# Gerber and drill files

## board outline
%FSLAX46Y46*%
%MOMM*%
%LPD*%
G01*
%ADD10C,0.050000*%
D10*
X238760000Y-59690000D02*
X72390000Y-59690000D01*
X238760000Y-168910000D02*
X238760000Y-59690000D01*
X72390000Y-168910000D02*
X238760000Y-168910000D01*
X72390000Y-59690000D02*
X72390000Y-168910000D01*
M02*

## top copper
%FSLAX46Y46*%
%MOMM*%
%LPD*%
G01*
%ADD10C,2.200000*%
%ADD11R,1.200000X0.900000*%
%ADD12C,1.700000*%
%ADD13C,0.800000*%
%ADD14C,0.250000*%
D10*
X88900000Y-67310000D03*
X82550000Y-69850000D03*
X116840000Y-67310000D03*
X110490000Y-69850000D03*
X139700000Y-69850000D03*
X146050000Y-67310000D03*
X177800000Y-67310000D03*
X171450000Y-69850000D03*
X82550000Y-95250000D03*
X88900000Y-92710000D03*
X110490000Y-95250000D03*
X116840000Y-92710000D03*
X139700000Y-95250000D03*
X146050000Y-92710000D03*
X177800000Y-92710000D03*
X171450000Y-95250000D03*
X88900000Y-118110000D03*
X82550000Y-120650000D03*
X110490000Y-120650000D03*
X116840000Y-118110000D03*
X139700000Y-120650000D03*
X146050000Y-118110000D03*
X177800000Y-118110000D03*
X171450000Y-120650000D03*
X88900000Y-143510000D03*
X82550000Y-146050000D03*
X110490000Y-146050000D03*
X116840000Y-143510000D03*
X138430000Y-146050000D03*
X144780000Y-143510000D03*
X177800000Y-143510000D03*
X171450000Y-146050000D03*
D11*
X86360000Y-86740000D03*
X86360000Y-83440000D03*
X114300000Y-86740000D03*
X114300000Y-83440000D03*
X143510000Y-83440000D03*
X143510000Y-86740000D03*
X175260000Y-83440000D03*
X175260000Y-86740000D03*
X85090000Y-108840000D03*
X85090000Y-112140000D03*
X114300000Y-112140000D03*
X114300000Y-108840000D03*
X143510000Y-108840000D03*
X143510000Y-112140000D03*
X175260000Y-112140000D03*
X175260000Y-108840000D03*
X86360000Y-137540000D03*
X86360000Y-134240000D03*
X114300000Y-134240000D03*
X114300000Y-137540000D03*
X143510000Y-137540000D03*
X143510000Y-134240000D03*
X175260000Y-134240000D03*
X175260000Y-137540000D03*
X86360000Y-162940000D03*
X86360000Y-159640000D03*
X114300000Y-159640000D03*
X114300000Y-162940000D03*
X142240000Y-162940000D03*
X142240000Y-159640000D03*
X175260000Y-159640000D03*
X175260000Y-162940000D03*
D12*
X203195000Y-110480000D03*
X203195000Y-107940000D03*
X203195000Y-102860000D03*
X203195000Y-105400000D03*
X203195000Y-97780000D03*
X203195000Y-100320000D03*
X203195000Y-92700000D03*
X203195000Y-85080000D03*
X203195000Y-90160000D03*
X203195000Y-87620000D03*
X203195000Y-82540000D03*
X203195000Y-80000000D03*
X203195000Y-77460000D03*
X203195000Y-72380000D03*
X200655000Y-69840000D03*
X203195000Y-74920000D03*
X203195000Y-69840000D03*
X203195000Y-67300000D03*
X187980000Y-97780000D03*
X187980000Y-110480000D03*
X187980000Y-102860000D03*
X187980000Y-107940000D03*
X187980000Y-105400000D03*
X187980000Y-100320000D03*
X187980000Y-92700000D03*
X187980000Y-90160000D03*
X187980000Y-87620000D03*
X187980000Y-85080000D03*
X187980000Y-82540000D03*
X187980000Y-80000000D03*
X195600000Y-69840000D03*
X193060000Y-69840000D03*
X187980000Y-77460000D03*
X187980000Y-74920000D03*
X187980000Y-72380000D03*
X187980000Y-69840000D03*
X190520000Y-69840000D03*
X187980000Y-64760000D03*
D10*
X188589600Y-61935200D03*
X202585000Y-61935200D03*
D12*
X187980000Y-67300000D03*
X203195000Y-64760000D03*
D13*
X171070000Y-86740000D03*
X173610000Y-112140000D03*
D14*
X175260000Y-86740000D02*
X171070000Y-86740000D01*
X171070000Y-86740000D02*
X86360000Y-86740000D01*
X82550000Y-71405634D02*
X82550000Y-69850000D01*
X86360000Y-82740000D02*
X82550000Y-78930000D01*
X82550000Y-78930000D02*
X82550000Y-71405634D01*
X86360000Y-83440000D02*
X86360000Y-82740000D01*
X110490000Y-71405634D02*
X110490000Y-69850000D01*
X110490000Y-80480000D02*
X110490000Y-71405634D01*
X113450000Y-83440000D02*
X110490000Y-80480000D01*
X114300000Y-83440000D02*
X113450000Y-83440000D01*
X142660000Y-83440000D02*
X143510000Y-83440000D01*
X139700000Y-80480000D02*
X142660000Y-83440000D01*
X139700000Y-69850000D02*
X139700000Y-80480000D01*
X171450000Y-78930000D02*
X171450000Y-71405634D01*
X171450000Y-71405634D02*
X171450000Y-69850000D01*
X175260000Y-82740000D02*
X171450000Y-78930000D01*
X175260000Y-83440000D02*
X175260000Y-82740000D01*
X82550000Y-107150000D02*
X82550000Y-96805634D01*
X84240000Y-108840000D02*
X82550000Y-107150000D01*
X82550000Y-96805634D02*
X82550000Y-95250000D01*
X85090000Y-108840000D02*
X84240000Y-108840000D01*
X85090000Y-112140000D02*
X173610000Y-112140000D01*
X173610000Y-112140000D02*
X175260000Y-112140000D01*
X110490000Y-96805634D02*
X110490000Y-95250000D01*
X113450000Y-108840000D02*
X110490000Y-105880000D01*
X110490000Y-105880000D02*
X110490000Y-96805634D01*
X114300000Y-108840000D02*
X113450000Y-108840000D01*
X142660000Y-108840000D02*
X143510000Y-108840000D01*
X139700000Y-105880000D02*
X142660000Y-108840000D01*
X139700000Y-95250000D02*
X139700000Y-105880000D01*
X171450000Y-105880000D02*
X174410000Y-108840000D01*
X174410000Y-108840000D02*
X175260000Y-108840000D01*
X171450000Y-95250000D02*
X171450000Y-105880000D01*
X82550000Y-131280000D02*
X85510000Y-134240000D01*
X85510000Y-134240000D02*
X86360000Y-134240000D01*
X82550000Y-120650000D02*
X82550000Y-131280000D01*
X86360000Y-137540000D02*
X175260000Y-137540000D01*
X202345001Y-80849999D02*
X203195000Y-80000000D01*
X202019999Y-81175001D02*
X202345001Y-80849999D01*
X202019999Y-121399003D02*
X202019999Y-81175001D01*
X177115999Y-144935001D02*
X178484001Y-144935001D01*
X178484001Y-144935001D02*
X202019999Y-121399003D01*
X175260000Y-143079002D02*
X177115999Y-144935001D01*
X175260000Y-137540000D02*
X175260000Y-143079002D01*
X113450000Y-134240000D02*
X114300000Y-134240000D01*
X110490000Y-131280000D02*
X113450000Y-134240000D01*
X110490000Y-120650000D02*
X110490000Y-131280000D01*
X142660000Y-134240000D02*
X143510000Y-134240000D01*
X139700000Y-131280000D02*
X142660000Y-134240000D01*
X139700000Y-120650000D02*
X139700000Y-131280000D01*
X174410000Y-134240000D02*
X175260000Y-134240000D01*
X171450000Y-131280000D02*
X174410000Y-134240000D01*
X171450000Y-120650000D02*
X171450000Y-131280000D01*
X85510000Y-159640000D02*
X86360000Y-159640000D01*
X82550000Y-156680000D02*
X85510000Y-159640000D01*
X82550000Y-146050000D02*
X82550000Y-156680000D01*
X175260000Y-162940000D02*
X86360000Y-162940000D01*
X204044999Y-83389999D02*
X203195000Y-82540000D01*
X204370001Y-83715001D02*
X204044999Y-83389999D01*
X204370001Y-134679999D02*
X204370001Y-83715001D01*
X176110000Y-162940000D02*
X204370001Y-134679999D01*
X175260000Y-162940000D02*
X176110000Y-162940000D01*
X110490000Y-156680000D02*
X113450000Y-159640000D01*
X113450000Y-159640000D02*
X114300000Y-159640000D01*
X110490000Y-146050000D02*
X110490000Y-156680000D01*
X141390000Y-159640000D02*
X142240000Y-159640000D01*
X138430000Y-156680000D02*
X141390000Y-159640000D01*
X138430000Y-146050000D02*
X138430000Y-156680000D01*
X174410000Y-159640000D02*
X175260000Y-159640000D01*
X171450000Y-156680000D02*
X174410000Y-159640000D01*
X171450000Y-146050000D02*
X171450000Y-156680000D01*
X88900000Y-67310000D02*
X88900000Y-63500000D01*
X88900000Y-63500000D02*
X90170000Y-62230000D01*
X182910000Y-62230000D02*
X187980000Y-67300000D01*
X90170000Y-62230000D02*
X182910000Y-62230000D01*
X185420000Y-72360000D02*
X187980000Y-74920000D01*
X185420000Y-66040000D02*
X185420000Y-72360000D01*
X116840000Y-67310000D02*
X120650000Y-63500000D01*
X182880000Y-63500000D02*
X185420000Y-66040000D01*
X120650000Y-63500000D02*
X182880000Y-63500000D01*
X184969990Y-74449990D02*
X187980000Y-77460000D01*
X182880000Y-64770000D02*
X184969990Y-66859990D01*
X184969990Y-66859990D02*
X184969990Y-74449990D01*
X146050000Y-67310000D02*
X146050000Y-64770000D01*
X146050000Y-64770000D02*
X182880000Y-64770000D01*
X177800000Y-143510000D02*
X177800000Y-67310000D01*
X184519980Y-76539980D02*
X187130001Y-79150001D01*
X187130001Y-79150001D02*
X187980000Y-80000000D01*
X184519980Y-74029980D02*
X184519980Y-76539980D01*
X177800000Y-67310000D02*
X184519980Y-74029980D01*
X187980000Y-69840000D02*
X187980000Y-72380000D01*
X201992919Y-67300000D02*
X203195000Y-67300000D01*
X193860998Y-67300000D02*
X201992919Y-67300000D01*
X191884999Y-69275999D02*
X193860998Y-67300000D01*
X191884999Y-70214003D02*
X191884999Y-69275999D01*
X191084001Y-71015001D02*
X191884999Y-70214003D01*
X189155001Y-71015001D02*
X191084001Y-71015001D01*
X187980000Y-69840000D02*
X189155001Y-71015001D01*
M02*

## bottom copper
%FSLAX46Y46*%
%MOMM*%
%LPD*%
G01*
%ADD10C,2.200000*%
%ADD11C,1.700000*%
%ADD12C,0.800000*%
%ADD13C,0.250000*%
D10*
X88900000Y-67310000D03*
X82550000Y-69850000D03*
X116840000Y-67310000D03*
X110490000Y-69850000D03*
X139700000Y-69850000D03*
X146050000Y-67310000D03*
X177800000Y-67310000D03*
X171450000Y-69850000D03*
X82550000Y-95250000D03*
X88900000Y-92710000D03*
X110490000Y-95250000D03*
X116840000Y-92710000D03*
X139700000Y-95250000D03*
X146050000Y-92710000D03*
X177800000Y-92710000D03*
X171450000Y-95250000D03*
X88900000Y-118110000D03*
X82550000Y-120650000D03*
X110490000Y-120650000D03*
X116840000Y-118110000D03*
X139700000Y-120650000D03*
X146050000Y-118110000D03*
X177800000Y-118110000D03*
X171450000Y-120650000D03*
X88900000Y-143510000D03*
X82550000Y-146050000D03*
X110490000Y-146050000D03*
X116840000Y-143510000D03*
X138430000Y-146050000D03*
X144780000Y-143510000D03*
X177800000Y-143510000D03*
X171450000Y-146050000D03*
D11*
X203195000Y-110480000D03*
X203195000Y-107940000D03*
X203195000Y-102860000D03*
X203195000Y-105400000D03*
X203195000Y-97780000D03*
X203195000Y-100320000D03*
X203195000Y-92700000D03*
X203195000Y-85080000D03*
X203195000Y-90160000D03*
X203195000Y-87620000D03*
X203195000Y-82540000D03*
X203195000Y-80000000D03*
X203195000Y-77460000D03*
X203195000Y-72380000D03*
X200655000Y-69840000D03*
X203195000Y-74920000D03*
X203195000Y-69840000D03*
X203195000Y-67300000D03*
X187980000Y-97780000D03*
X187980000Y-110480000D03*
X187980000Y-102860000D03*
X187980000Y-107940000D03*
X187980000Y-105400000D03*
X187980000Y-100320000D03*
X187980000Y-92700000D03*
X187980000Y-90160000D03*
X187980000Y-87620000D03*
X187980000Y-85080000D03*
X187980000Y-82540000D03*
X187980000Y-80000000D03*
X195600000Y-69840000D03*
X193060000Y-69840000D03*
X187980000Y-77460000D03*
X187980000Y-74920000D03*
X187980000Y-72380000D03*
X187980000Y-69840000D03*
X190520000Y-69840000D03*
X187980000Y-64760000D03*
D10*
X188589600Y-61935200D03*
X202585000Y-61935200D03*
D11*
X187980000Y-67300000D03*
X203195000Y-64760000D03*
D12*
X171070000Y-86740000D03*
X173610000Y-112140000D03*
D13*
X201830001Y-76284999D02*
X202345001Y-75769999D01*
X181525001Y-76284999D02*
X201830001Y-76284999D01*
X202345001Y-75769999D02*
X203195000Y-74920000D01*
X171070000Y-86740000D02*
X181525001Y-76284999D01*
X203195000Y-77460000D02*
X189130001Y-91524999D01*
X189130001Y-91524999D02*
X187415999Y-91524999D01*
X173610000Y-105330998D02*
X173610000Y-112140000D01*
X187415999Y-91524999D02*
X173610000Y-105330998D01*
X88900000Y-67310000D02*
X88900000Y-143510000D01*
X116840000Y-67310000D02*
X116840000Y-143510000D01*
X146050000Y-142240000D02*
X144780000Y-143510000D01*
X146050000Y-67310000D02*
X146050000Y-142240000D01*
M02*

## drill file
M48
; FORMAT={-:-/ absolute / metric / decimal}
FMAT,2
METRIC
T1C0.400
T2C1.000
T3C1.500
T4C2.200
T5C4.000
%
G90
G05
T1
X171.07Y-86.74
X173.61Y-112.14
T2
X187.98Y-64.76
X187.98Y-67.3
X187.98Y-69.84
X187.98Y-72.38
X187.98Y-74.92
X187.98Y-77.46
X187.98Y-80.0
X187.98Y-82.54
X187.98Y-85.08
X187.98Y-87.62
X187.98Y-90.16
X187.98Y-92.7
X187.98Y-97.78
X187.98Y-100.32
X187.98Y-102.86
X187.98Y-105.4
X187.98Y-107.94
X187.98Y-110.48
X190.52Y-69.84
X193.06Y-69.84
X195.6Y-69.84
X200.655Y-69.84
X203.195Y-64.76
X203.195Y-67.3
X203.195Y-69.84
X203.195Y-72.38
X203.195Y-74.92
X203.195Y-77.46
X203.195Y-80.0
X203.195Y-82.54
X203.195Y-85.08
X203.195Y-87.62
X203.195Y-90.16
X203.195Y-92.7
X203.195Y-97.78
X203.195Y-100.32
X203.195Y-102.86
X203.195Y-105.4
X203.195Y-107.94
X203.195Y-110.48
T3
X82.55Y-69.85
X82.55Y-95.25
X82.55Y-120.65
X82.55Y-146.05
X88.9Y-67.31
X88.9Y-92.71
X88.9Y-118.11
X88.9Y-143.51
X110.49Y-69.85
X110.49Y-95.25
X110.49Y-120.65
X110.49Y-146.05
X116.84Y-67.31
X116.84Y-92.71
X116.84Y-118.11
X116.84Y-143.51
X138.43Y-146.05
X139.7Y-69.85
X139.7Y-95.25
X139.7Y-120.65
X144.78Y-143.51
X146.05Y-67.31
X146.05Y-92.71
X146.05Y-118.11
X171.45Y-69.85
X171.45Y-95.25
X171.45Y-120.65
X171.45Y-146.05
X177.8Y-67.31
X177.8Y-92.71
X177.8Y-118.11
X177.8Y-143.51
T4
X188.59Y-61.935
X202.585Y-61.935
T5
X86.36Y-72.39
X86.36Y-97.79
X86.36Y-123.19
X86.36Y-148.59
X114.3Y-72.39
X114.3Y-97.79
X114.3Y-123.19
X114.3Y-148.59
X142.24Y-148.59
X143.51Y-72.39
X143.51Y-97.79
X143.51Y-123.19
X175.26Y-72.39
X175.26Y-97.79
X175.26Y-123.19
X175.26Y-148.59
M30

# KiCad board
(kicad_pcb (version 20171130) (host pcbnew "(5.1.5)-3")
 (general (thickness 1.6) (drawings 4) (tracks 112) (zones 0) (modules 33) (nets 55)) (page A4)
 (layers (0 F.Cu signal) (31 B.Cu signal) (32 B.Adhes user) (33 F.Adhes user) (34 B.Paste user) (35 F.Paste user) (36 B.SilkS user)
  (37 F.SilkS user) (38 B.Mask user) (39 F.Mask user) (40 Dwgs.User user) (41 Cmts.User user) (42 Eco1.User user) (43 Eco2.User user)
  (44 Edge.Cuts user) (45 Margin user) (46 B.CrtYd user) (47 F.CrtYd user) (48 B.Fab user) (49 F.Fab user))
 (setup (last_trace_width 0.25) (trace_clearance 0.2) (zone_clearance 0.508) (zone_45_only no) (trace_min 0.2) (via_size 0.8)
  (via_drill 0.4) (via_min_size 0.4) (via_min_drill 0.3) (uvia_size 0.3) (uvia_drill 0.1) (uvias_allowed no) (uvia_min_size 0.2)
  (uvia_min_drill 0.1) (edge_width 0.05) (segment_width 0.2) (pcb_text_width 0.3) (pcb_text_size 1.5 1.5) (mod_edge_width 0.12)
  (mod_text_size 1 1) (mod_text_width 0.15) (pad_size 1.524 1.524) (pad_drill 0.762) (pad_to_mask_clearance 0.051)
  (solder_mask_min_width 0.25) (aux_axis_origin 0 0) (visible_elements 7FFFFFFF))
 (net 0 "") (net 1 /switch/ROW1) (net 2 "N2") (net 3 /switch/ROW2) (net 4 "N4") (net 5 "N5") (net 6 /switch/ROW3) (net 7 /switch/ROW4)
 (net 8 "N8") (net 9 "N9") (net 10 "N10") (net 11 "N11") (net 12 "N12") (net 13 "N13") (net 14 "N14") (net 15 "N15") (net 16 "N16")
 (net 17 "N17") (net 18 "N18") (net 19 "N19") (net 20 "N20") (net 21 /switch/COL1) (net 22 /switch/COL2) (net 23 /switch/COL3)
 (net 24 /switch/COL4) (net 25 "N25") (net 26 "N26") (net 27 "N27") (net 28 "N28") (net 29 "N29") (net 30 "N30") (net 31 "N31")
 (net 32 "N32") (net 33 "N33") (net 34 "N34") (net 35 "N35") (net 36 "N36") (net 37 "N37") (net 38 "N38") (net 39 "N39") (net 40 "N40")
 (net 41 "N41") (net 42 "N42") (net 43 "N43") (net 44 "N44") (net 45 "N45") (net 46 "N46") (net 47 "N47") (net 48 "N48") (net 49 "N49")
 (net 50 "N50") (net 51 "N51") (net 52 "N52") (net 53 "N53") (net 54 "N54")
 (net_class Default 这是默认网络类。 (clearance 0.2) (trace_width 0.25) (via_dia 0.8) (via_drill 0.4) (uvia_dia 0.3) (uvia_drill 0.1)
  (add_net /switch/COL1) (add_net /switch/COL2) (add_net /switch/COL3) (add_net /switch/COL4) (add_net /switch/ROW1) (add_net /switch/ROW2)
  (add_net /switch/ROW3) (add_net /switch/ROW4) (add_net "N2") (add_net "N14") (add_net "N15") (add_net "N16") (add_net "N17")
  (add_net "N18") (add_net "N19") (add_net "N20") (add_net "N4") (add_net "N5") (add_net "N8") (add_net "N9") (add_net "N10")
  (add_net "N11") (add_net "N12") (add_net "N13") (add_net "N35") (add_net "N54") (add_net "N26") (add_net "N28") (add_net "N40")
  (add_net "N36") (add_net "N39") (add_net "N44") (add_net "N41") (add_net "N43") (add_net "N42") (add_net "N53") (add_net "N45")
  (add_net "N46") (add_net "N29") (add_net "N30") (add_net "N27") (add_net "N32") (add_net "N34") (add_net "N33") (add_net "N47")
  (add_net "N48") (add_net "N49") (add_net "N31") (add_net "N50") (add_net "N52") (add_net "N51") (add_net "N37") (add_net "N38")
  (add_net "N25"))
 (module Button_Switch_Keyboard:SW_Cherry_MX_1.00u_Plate (layer F.Cu) (at 88.9 67.31)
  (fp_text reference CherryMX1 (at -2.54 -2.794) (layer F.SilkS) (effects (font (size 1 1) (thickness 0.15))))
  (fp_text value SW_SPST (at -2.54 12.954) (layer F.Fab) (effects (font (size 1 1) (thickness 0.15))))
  (pad 1 thru_hole circle (at 0 0) (size 2.2 2.2) (drill 1.5) (layers *.Cu *.Mask) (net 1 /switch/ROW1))
  (pad 2 thru_hole circle (at -6.35 2.54) (size 2.2 2.2) (drill 1.5) (layers *.Cu *.Mask) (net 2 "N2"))
  (pad "" np_thru_hole circle (at -2.54 5.08) (size 4 4) (drill 4) (layers *.Cu *.Mask)))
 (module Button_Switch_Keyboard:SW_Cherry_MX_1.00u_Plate (layer F.Cu) (at 116.84 67.31)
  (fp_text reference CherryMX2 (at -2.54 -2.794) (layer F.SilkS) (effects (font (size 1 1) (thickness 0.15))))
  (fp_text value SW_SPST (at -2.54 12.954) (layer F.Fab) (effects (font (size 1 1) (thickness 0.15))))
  (pad 1 thru_hole circle (at 0 0) (size 2.2 2.2) (drill 1.5) (layers *.Cu *.Mask) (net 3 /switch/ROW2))
  (pad 2 thru_hole circle (at -6.35 2.54) (size 2.2 2.2) (drill 1.5) (layers *.Cu *.Mask) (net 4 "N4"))
  (pad "" np_thru_hole circle (at -2.54 5.08) (size 4 4) (drill 4) (layers *.Cu *.Mask)))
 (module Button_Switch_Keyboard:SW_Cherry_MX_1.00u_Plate (layer F.Cu) (at 146.05 67.31)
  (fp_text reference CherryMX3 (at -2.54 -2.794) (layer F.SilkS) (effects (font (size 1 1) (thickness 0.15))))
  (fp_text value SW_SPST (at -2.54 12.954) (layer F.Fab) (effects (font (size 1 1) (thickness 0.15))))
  (pad "" np_thru_hole circle (at -2.54 5.08) (size 4 4) (drill 4) (layers *.Cu *.Mask))
  (pad 2 thru_hole circle (at -6.35 2.54) (size 2.2 2.2) (drill 1.5) (layers *.Cu *.Mask) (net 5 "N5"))
  (pad 1 thru_hole circle (at 0 0) (size 2.2 2.2) (drill 1.5) (layers *.Cu *.Mask) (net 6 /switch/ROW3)))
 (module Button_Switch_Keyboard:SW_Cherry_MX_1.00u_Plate (layer F.Cu) (at 177.8 67.31)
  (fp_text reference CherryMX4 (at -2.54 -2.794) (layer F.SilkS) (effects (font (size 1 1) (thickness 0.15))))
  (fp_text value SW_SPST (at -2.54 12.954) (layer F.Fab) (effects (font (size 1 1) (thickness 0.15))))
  (pad 1 thru_hole circle (at 0 0) (size 2.2 2.2) (drill 1.5) (layers *.Cu *.Mask) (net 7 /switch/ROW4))
  (pad 2 thru_hole circle (at -6.35 2.54) (size 2.2 2.2) (drill 1.5) (layers *.Cu *.Mask) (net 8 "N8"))
  (pad "" np_thru_hole circle (at -2.54 5.08) (size 4 4) (drill 4) (layers *.Cu *.Mask)))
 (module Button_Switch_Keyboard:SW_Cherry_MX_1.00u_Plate (layer F.Cu) (at 88.9 92.71)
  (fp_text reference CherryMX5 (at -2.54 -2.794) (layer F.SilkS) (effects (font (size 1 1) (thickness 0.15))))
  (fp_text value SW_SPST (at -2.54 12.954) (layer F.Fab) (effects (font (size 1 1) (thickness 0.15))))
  (pad "" np_thru_hole circle (at -2.54 5.08) (size 4 4) (drill 4) (layers *.Cu *.Mask))
  (pad 2 thru_hole circle (at -6.35 2.54) (size 2.2 2.2) (drill 1.5) (layers *.Cu *.Mask) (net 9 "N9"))
  (pad 1 thru_hole circle (at 0 0) (size 2.2 2.2) (drill 1.5) (layers *.Cu *.Mask) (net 1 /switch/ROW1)))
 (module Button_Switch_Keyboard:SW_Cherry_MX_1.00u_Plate (layer F.Cu) (at 116.84 92.71)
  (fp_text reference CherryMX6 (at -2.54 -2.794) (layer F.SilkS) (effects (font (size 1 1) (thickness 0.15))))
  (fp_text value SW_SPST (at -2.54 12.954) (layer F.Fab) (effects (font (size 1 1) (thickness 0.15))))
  (pad "" np_thru_hole circle (at -2.54 5.08) (size 4 4) (drill 4) (layers *.Cu *.Mask))
  (pad 2 thru_hole circle (at -6.35 2.54) (size 2.2 2.2) (drill 1.5) (layers *.Cu *.Mask) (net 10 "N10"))
  (pad 1 thru_hole circle (at 0 0) (size 2.2 2.2) (drill 1.5) (layers *.Cu *.Mask) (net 3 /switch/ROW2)))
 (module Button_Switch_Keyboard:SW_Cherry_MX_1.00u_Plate (layer F.Cu) (at 146.05 92.71)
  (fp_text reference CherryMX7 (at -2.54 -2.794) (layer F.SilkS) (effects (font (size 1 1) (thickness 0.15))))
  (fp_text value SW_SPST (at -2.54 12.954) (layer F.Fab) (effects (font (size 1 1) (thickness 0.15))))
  (pad "" np_thru_hole circle (at -2.54 5.08) (size 4 4) (drill 4) (layers *.Cu *.Mask))
  (pad 2 thru_hole circle (at -6.35 2.54) (size 2.2 2.2) (drill 1.5) (layers *.Cu *.Mask) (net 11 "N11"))
  (pad 1 thru_hole circle (at 0 0) (size 2.2 2.2) (drill 1.5) (layers *.Cu *.Mask) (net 6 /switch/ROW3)))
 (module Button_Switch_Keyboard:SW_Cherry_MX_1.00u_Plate (layer F.Cu) (at 177.8 92.71)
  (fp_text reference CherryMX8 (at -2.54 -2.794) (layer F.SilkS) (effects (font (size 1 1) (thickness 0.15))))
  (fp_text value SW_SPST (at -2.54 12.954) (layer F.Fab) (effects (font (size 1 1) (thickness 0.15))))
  (pad 1 thru_hole circle (at 0 0) (size 2.2 2.2) (drill 1.5) (layers *.Cu *.Mask) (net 7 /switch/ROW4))
  (pad 2 thru_hole circle (at -6.35 2.54) (size 2.2 2.2) (drill 1.5) (layers *.Cu *.Mask) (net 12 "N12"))
  (pad "" np_thru_hole circle (at -2.54 5.08) (size 4 4) (drill 4) (layers *.Cu *.Mask)))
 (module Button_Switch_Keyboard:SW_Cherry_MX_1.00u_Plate (layer F.Cu) (at 88.9 118.11)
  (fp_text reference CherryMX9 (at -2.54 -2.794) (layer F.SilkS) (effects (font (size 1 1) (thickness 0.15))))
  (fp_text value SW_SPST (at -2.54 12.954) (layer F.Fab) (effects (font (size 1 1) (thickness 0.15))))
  (pad 1 thru_hole circle (at 0 0) (size 2.2 2.2) (drill 1.5) (layers *.Cu *.Mask) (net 1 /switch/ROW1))
  (pad 2 thru_hole circle (at -6.35 2.54) (size 2.2 2.2) (drill 1.5) (layers *.Cu *.Mask) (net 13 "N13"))
  (pad "" np_thru_hole circle (at -2.54 5.08) (size 4 4) (drill 4) (layers *.Cu *.Mask)))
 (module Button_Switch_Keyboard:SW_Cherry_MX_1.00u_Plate (layer F.Cu) (at 116.84 118.11)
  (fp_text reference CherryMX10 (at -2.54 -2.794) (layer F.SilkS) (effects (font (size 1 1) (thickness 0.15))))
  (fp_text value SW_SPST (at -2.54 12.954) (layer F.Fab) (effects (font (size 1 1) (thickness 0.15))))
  (pad "" np_thru_hole circle (at -2.54 5.08) (size 4 4) (drill 4) (layers *.Cu *.Mask))
  (pad 2 thru_hole circle (at -6.35 2.54) (size 2.2 2.2) (drill 1.5) (layers *.Cu *.Mask) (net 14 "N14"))
  (pad 1 thru_hole circle (at 0 0) (size 2.2 2.2) (drill 1.5) (layers *.Cu *.Mask) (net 3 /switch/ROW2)))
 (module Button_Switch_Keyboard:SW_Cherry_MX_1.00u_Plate (layer F.Cu) (at 146.05 118.11)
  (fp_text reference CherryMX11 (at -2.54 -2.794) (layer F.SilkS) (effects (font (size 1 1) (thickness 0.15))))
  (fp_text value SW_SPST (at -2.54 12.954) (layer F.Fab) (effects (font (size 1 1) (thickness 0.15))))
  (pad "" np_thru_hole circle (at -2.54 5.08) (size 4 4) (drill 4) (layers *.Cu *.Mask))
  (pad 2 thru_hole circle (at -6.35 2.54) (size 2.2 2.2) (drill 1.5) (layers *.Cu *.Mask) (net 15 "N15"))
  (pad 1 thru_hole circle (at 0 0) (size 2.2 2.2) (drill 1.5) (layers *.Cu *.Mask) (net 6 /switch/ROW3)))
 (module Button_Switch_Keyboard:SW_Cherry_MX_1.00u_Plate (layer F.Cu) (at 177.8 118.11)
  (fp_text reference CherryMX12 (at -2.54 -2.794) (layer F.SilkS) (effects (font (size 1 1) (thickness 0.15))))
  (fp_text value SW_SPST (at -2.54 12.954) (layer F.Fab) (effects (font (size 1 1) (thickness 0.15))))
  (pad 1 thru_hole circle (at 0 0) (size 2.2 2.2) (drill 1.5) (layers *.Cu *.Mask) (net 7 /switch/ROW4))
  (pad 2 thru_hole circle (at -6.35 2.54) (size 2.2 2.2) (drill 1.5) (layers *.Cu *.Mask) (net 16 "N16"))
  (pad "" np_thru_hole circle (at -2.54 5.08) (size 4 4) (drill 4) (layers *.Cu *.Mask)))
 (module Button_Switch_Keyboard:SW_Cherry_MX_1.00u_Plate (layer F.Cu) (at 88.9 143.51)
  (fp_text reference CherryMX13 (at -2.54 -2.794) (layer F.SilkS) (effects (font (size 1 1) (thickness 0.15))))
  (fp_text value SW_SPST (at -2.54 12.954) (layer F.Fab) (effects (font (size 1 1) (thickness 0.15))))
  (pad 1 thru_hole circle (at 0 0) (size 2.2 2.2) (drill 1.5) (layers *.Cu *.Mask) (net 1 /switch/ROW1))
  (pad 2 thru_hole circle (at -6.35 2.54) (size 2.2 2.2) (drill 1.5) (layers *.Cu *.Mask) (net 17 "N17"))
  (pad "" np_thru_hole circle (at -2.54 5.08) (size 4 4) (drill 4) (layers *.Cu *.Mask)))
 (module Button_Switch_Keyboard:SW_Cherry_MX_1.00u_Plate (layer F.Cu) (at 116.84 143.51)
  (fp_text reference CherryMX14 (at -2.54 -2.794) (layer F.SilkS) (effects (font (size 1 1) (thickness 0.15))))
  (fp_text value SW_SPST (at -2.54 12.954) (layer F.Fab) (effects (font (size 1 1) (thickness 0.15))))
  (pad "" np_thru_hole circle (at -2.54 5.08) (size 4 4) (drill 4) (layers *.Cu *.Mask))
  (pad 2 thru_hole circle (at -6.35 2.54) (size 2.2 2.2) (drill 1.5) (layers *.Cu *.Mask) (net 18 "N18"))
  (pad 1 thru_hole circle (at 0 0) (size 2.2 2.2) (drill 1.5) (layers *.Cu *.Mask) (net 3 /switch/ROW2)))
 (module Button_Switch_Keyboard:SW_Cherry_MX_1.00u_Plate (layer F.Cu) (at 144.78 143.51)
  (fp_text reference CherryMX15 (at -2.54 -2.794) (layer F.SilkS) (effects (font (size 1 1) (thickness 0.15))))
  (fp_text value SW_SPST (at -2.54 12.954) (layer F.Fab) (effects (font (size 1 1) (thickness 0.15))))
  (pad "" np_thru_hole circle (at -2.54 5.08) (size 4 4) (drill 4) (layers *.Cu *.Mask))
  (pad 2 thru_hole circle (at -6.35 2.54) (size 2.2 2.2) (drill 1.5) (layers *.Cu *.Mask) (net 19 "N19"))
  (pad 1 thru_hole circle (at 0 0) (size 2.2 2.2) (drill 1.5) (layers *.Cu *.Mask) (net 6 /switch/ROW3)))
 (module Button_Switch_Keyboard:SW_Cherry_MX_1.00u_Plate (layer F.Cu) (at 177.8 143.51)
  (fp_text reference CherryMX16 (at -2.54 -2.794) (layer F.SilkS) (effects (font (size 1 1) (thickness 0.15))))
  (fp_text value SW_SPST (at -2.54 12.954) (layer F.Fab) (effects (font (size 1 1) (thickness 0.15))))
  (pad 1 thru_hole circle (at 0 0) (size 2.2 2.2) (drill 1.5) (layers *.Cu *.Mask) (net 7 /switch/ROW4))
  (pad 2 thru_hole circle (at -6.35 2.54) (size 2.2 2.2) (drill 1.5) (layers *.Cu *.Mask) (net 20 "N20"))
  (pad "" np_thru_hole circle (at -2.54 5.08) (size 4 4) (drill 4) (layers *.Cu *.Mask)))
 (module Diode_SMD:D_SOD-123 (layer F.Cu) (at 86.36 85.09 90)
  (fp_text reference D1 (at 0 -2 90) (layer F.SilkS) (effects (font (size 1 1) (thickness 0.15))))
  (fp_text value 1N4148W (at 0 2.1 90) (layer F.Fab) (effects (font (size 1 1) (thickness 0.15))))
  (pad 1 smd rect (at -1.65 0 90) (size 0.9 1.2) (layers F.Cu F.Paste F.Mask) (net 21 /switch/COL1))
  (pad 2 smd rect (at 1.65 0 90) (size 0.9 1.2) (layers F.Cu F.Paste F.Mask) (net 2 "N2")))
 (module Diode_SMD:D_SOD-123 (layer F.Cu) (at 114.3 85.09 90)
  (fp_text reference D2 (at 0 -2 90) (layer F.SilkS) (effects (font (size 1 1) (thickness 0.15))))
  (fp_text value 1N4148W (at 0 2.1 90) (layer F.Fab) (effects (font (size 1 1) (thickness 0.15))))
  (pad 1 smd rect (at -1.65 0 90) (size 0.9 1.2) (layers F.Cu F.Paste F.Mask) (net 21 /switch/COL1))
  (pad 2 smd rect (at 1.65 0 90) (size 0.9 1.2) (layers F.Cu F.Paste F.Mask) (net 4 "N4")))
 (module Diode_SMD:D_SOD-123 (layer F.Cu) (at 143.51 85.09 90)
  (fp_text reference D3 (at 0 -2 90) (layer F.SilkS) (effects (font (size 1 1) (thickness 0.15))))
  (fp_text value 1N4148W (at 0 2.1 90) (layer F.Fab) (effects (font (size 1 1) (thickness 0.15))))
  (pad 2 smd rect (at 1.65 0 90) (size 0.9 1.2) (layers F.Cu F.Paste F.Mask) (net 5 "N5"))
  (pad 1 smd rect (at -1.65 0 90) (size 0.9 1.2) (layers F.Cu F.Paste F.Mask) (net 21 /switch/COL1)))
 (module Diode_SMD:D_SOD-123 (layer F.Cu) (at 175.26 85.09 90)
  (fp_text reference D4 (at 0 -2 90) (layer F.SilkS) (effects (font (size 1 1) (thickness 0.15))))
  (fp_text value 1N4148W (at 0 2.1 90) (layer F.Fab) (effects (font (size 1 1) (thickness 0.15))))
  (pad 2 smd rect (at 1.65 0 90) (size 0.9 1.2) (layers F.Cu F.Paste F.Mask) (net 8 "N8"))
  (pad 1 smd rect (at -1.65 0 90) (size 0.9 1.2) (layers F.Cu F.Paste F.Mask) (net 21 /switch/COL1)))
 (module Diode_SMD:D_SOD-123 (layer F.Cu) (at 85.09 110.49 90)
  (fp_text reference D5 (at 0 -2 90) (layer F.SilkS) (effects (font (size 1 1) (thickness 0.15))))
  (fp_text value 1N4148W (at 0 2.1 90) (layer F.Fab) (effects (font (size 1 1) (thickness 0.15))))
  (pad 2 smd rect (at 1.65 0 90) (size 0.9 1.2) (layers F.Cu F.Paste F.Mask) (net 9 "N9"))
  (pad 1 smd rect (at -1.65 0 90) (size 0.9 1.2) (layers F.Cu F.Paste F.Mask) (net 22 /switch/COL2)))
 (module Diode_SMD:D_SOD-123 (layer F.Cu) (at 114.3 110.49 90)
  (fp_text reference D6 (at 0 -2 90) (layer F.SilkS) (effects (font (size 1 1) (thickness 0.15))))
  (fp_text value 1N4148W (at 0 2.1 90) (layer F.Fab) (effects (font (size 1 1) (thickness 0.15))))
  (pad 1 smd rect (at -1.65 0 90) (size 0.9 1.2) (layers F.Cu F.Paste F.Mask) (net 22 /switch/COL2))
  (pad 2 smd rect (at 1.65 0 90) (size 0.9 1.2) (layers F.Cu F.Paste F.Mask) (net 10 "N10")))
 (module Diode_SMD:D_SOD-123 (layer F.Cu) (at 143.51 110.49 90)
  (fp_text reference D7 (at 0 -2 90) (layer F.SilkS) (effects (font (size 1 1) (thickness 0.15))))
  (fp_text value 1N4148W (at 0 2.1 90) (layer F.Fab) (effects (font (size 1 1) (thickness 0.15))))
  (pad 2 smd rect (at 1.65 0 90) (size 0.9 1.2) (layers F.Cu F.Paste F.Mask) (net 11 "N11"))
  (pad 1 smd rect (at -1.65 0 90) (size 0.9 1.2) (layers F.Cu F.Paste F.Mask) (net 22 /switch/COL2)))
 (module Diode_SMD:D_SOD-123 (layer F.Cu) (at 175.26 110.49 90)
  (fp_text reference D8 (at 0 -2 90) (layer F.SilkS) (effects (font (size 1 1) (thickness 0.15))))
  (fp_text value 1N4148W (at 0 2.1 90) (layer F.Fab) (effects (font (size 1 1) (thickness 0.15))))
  (pad 1 smd rect (at -1.65 0 90) (size 0.9 1.2) (layers F.Cu F.Paste F.Mask) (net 22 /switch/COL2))
  (pad 2 smd rect (at 1.65 0 90) (size 0.9 1.2) (layers F.Cu F.Paste F.Mask) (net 12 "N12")))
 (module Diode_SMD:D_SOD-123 (layer F.Cu) (at 86.36 135.89 90)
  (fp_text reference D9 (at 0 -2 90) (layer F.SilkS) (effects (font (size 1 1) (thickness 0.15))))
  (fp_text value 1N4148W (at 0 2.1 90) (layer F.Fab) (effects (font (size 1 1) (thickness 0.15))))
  (pad 1 smd rect (at -1.65 0 90) (size 0.9 1.2) (layers F.Cu F.Paste F.Mask) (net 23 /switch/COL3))
  (pad 2 smd rect (at 1.65 0 90) (size 0.9 1.2) (layers F.Cu F.Paste F.Mask) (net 13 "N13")))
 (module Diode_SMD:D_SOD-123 (layer F.Cu) (at 114.3 135.89 90)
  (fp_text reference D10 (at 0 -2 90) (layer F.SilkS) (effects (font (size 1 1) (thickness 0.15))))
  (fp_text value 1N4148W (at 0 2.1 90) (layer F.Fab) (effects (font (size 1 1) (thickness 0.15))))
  (pad 2 smd rect (at 1.65 0 90) (size 0.9 1.2) (layers F.Cu F.Paste F.Mask) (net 14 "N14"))
  (pad 1 smd rect (at -1.65 0 90) (size 0.9 1.2) (layers F.Cu F.Paste F.Mask) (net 23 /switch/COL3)))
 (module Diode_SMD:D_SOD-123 (layer F.Cu) (at 143.51 135.89 90)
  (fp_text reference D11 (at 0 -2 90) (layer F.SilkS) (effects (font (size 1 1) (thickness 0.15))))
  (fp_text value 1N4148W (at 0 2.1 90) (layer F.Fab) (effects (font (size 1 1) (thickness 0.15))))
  (pad 1 smd rect (at -1.65 0 90) (size 0.9 1.2) (layers F.Cu F.Paste F.Mask) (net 23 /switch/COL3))
  (pad 2 smd rect (at 1.65 0 90) (size 0.9 1.2) (layers F.Cu F.Paste F.Mask) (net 15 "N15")))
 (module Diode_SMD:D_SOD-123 (layer F.Cu) (at 175.26 135.89 90)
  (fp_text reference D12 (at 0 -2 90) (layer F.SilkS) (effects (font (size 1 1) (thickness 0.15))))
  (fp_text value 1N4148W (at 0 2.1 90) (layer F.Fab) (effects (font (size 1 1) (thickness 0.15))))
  (pad 2 smd rect (at 1.65 0 90) (size 0.9 1.2) (layers F.Cu F.Paste F.Mask) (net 16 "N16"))
  (pad 1 smd rect (at -1.65 0 90) (size 0.9 1.2) (layers F.Cu F.Paste F.Mask) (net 23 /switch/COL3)))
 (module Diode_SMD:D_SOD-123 (layer F.Cu) (at 86.36 161.29 90)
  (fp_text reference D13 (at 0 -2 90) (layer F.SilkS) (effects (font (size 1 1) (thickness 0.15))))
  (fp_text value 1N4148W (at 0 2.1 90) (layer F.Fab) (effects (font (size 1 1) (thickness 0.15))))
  (pad 1 smd rect (at -1.65 0 90) (size 0.9 1.2) (layers F.Cu F.Paste F.Mask) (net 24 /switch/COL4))
  (pad 2 smd rect (at 1.65 0 90) (size 0.9 1.2) (layers F.Cu F.Paste F.Mask) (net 17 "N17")))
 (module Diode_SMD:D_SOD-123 (layer F.Cu) (at 114.3 161.29 90)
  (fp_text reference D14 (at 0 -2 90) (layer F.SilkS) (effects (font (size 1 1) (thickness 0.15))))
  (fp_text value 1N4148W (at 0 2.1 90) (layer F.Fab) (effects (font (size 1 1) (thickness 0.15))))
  (pad 2 smd rect (at 1.65 0 90) (size 0.9 1.2) (layers F.Cu F.Paste F.Mask) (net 18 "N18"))
  (pad 1 smd rect (at -1.65 0 90) (size 0.9 1.2) (layers F.Cu F.Paste F.Mask) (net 24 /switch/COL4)))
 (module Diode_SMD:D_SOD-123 (layer F.Cu) (at 142.24 161.29 90)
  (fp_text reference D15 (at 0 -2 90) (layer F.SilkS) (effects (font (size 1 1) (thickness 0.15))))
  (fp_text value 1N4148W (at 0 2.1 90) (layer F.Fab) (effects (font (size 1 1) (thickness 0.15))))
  (pad 1 smd rect (at -1.65 0 90) (size 0.9 1.2) (layers F.Cu F.Paste F.Mask) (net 24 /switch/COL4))
  (pad 2 smd rect (at 1.65 0 90) (size 0.9 1.2) (layers F.Cu F.Paste F.Mask) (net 19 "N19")))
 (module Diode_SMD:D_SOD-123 (layer F.Cu) (at 175.26 161.29 90)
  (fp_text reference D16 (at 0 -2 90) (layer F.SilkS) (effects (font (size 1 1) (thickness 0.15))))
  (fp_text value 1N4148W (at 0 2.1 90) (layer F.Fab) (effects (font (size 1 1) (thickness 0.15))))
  (pad 2 smd rect (at 1.65 0 90) (size 0.9 1.2) (layers F.Cu F.Paste F.Mask) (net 20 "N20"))
  (pad 1 smd rect (at -1.65 0 90) (size 0.9 1.2) (layers F.Cu F.Paste F.Mask) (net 24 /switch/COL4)))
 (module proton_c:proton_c (layer F.Cu) (at 195.58 80.01)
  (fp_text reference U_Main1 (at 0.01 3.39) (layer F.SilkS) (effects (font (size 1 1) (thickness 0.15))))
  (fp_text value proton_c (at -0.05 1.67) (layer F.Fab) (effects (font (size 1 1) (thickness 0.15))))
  (pad RST thru_hole circle (at 7.615 30.47) (size 1.7 1.7) (drill 1) (layers *.Cu *.Mask) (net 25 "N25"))
  (pad A13 thru_hole circle (at 7.615 27.93) (size 1.7 1.7) (drill 1) (layers *.Cu *.Mask) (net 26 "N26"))
  (pad B12 thru_hole circle (at 7.615 22.85) (size 1.7 1.7) (drill 1) (layers *.Cu *.Mask) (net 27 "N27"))
  (pad A14 thru_hole circle (at 7.615 25.39) (size 1.7 1.7) (drill 1) (layers *.Cu *.Mask) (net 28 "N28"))
  (pad B10 thru_hole circle (at 7.615 17.77) (size 1.7 1.7) (drill 1) (layers *.Cu *.Mask) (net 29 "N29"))
  (pad B11 thru_hole circle (at 7.615 20.31) (size 1.7 1.7) (drill 1) (layers *.Cu *.Mask) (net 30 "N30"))
  (pad B9 thru_hole circle (at 7.615 12.69) (size 1.7 1.7) (drill 1) (layers *.Cu *.Mask) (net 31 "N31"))
  (pad B13 thru_hole circle (at 7.615 5.07) (size 1.7 1.7) (drill 1) (layers *.Cu *.Mask) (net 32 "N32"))
  (pad B15 thru_hole circle (at 7.615 10.15) (size 1.7 1.7) (drill 1) (layers *.Cu *.Mask) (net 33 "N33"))
  (pad B14 thru_hole circle (at 7.615 7.61) (size 1.7 1.7) (drill 1) (layers *.Cu *.Mask) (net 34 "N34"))
  (pad B8 thru_hole circle (at 7.615 2.53) (size 1.7 1.7) (drill 1) (layers *.Cu *.Mask) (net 24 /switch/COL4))
  (pad A0 thru_hole circle (at 7.615 -0.01) (size 1.7 1.7) (drill 1) (layers *.Cu *.Mask) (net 23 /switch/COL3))
  (pad A1 thru_hole circle (at 7.615 -2.55) (size 1.7 1.7) (drill 1) (layers *.Cu *.Mask) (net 22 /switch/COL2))
  (pad 3.3V thru_hole circle (at 7.615 -7.63) (size 1.7 1.7) (drill 1) (layers *.Cu *.Mask) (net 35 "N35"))
  (pad A3|5v thru_hole circle (at 5.075 -10.17) (size 1.7 1.7) (drill 1) (layers *.Cu *.Mask) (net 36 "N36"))
  (pad A2 thru_hole circle (at 7.615 -5.09) (size 1.7 1.7) (drill 1) (layers *.Cu *.Mask) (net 21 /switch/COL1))
  (pad DFU thru_hole circle (at 7.615 -10.17) (size 1.7 1.7) (drill 1) (layers *.Cu *.Mask) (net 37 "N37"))
  (pad GND thru_hole circle (at 7.615 -12.71) (size 1.7 1.7) (drill 1) (layers *.Cu *.Mask) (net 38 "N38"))
  (pad A4 thru_hole circle (at -7.6 17.77) (size 1.7 1.7) (drill 1) (layers *.Cu *.Mask) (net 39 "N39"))
  (pad A15 thru_hole circle (at -7.6 30.47) (size 1.7 1.7) (drill 1) (layers *.Cu *.Mask) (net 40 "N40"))
  (pad A6 thru_hole circle (at -7.6 22.85) (size 1.7 1.7) (drill 1) (layers *.Cu *.Mask) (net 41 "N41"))
  (pad A8 thru_hole circle (at -7.6 27.93) (size 1.7 1.7) (drill 1) (layers *.Cu *.Mask) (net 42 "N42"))
  (pad A7 thru_hole circle (at -7.6 25.39) (size 1.7 1.7) (drill 1) (layers *.Cu *.Mask) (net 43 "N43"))
  (pad A5 thru_hole circle (at -7.6 20.31) (size 1.7 1.7) (drill 1) (layers *.Cu *.Mask) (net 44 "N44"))
  (pad B0 thru_hole circle (at -7.6 12.69) (size 1.7 1.7) (drill 1) (layers *.Cu *.Mask) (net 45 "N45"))
  (pad B1 thru_hole circle (at -7.6 10.15) (size 1.7 1.7) (drill 1) (layers *.Cu *.Mask) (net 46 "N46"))
  (pad B2 thru_hole circle (at -7.6 7.61) (size 1.7 1.7) (drill 1) (layers *.Cu *.Mask) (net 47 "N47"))
  (pad B3 thru_hole circle (at -7.6 5.07) (size 1.7 1.7) (drill 1) (layers *.Cu *.Mask) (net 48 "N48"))
  (pad B4 thru_hole circle (at -7.6 2.53) (size 1.7 1.7) (drill 1) (layers *.Cu *.Mask) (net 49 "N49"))
  (pad B5 thru_hole circle (at -7.6 -0.01) (size 1.7 1.7) (drill 1) (layers *.Cu *.Mask) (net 7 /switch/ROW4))
  (pad CHRG thru_hole circle (at 0.02 -10.17) (size 1.7 1.7) (drill 1) (layers *.Cu *.Mask) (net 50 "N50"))
  (pad D- thru_hole circle (at -2.52 -10.17) (size 1.7 1.7) (drill 1) (layers *.Cu *.Mask) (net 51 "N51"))
  (pad B6 thru_hole circle (at -7.6 -2.55) (size 1.7 1.7) (drill 1) (layers *.Cu *.Mask) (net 6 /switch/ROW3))
  (pad B7 thru_hole circle (at -7.6 -5.09) (size 1.7 1.7) (drill 1) (layers *.Cu *.Mask) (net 3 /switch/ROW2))
  (pad GND thru_hole circle (at -7.6 -7.63) (size 1.7 1.7) (drill 1) (layers *.Cu *.Mask) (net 38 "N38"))
  (pad GND thru_hole circle (at -7.6 -10.17) (size 1.7 1.7) (drill 1) (layers *.Cu *.Mask) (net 38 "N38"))
  (pad D+ thru_hole circle (at -5.06 -10.17) (size 1.7 1.7) (drill 1) (layers *.Cu *.Mask) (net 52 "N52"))
  (pad A9 thru_hole circle (at -7.6 -15.25) (size 1.7 1.7) (drill 1) (layers *.Cu *.Mask) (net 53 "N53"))
  (pad SCRE thru_hole circle (at -6.9904 -18.0748) (size 2.2 2.2) (drill 2.2) (layers *.Cu *.Mask))
  (pad SCRE thru_hole circle (at 7.005 -18.0748) (size 2.2 2.2) (drill 2.2) (layers *.Cu *.Mask))
  (pad A10 thru_hole circle (at -7.6 -12.71) (size 1.7 1.7) (drill 1) (layers *.Cu *.Mask) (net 1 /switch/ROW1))
  (pad 5V thru_hole circle (at 7.615 -15.25) (size 1.7 1.7) (drill 1) (layers *.Cu *.Mask) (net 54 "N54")))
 (gr_line (start 238.76 59.69) (end 72.39 59.69) (layer Edge.Cuts) (width 0.05))
 (gr_line (start 238.76 168.91) (end 238.76 59.69) (layer Edge.Cuts) (width 0.05))
 (gr_line (start 72.39 168.91) (end 238.76 168.91) (layer Edge.Cuts) (width 0.05))
 (gr_line (start 72.39 59.69) (end 72.39 168.91) (layer Edge.Cuts) (width 0.05))
 (segment (start 175.26 86.74) (end 171.07 86.74) (width 0.25) (layer F.Cu) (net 21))
 (segment (start 171.07 86.74) (end 86.36 86.74) (width 0.25) (layer F.Cu) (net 21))
 (via (at 171.07 86.74) (size 0.8) (drill 0.4) (layers F.Cu B.Cu) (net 21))
 (segment (start 201.830001 76.284999) (end 202.345001 75.769999) (width 0.25) (layer B.Cu) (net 21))
 (segment (start 181.525001 76.284999) (end 201.830001 76.284999) (width 0.25) (layer B.Cu) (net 21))
 (segment (start 202.345001 75.769999) (end 203.195 74.92) (width 0.25) (layer B.Cu) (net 21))
 (segment (start 171.07 86.74) (end 181.525001 76.284999) (width 0.25) (layer B.Cu) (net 21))
 (segment (start 82.55 71.405634) (end 82.55 69.85) (width 0.25) (layer F.Cu) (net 2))
 (segment (start 86.36 82.74) (end 82.55 78.93) (width 0.25) (layer F.Cu) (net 2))
 (segment (start 82.55 78.93) (end 82.55 71.405634) (width 0.25) (layer F.Cu) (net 2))
 (segment (start 86.36 83.44) (end 86.36 82.74) (width 0.25) (layer F.Cu) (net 2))
 (segment (start 110.49 71.405634) (end 110.49 69.85) (width 0.25) (layer F.Cu) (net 4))
 (segment (start 110.49 80.48) (end 110.49 71.405634) (width 0.25) (layer F.Cu) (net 4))
 (segment (start 113.45 83.44) (end 110.49 80.48) (width 0.25) (layer F.Cu) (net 4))
 (segment (start 114.3 83.44) (end 113.45 83.44) (width 0.25) (layer F.Cu) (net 4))
 (segment (start 142.66 83.44) (end 143.51 83.44) (width 0.25) (layer F.Cu) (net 5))
 (segment (start 139.7 80.48) (end 142.66 83.44) (width 0.25) (layer F.Cu) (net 5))
 (segment (start 139.7 69.85) (end 139.7 80.48) (width 0.25) (layer F.Cu) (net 5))
 (segment (start 171.45 78.93) (end 171.45 71.405634) (width 0.25) (layer F.Cu) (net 8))
 (segment (start 171.45 71.405634) (end 171.45 69.85) (width 0.25) (layer F.Cu) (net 8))
 (segment (start 175.26 82.74) (end 171.45 78.93) (width 0.25) (layer F.Cu) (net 8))
 (segment (start 175.26 83.44) (end 175.26 82.74) (width 0.25) (layer F.Cu) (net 8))
 (segment (start 82.55 107.15) (end 82.55 96.805634) (width 0.25) (layer F.Cu) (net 9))
 (segment (start 84.24 108.84) (end 82.55 107.15) (width 0.25) (layer F.Cu) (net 9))
 (segment (start 82.55 96.805634) (end 82.55 95.25) (width 0.25) (layer F.Cu) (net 9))
 (segment (start 85.09 108.84) (end 84.24 108.84) (width 0.25) (layer F.Cu) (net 9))
 (segment (start 85.09 112.14) (end 173.61 112.14) (width 0.25) (layer F.Cu) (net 22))
 (segment (start 203.195 77.46) (end 189.130001 91.524999) (width 0.25) (layer B.Cu) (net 22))
 (segment (start 189.130001 91.524999) (end 187.415999 91.524999) (width 0.25) (layer B.Cu) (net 22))
 (segment (start 173.61 112.14) (end 175.26 112.14) (width 0.25) (layer F.Cu) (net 22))
 (via (at 173.61 112.14) (size 0.8) (drill 0.4) (layers F.Cu B.Cu) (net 22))
 (segment (start 173.61 105.330998) (end 173.61 112.14) (width 0.25) (layer B.Cu) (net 22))
 (segment (start 187.415999 91.524999) (end 173.61 105.330998) (width 0.25) (layer B.Cu) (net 22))
 (segment (start 110.49 96.805634) (end 110.49 95.25) (width 0.25) (layer F.Cu) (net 10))
 (segment (start 113.45 108.84) (end 110.49 105.88) (width 0.25) (layer F.Cu) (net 10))
 (segment (start 110.49 105.88) (end 110.49 96.805634) (width 0.25) (layer F.Cu) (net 10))
 (segment (start 114.3 108.84) (end 113.45 108.84) (width 0.25) (layer F.Cu) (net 10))
 (segment (start 142.66 108.84) (end 143.51 108.84) (width 0.25) (layer F.Cu) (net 11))
 (segment (start 139.7 105.88) (end 142.66 108.84) (width 0.25) (layer F.Cu) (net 11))
 (segment (start 139.7 95.25) (end 139.7 105.88) (width 0.25) (layer F.Cu) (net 11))
 (segment (start 171.45 105.88) (end 174.41 108.84) (width 0.25) (layer F.Cu) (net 12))
 (segment (start 174.41 108.84) (end 175.26 108.84) (width 0.25) (layer F.Cu) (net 12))
 (segment (start 171.45 95.25) (end 171.45 105.88) (width 0.25) (layer F.Cu) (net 12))
 (segment (start 82.55 131.28) (end 85.51 134.24) (width 0.25) (layer F.Cu) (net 13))
 (segment (start 85.51 134.24) (end 86.36 134.24) (width 0.25) (layer F.Cu) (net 13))
 (segment (start 82.55 120.65) (end 82.55 131.28) (width 0.25) (layer F.Cu) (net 13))
 (segment (start 86.36 137.54) (end 175.26 137.54) (width 0.25) (layer F.Cu) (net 23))
 (segment (start 202.345001 80.849999) (end 203.195 80) (width 0.25) (layer F.Cu) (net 23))
 (segment (start 202.019999 81.175001) (end 202.345001 80.849999) (width 0.25) (layer F.Cu) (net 23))
 (segment (start 202.019999 121.399003) (end 202.019999 81.175001) (width 0.25) (layer F.Cu) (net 23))
 (segment (start 177.115999 144.935001) (end 178.484001 144.935001) (width 0.25) (layer F.Cu) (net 23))
 (segment (start 178.484001 144.935001) (end 202.019999 121.399003) (width 0.25) (layer F.Cu) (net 23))
 (segment (start 175.26 143.079002) (end 177.115999 144.935001) (width 0.25) (layer F.Cu) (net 23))
 (segment (start 175.26 137.54) (end 175.26 143.079002) (width 0.25) (layer F.Cu) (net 23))
 (segment (start 113.45 134.24) (end 114.3 134.24) (width 0.25) (layer F.Cu) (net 14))
 (segment (start 110.49 131.28) (end 113.45 134.24) (width 0.25) (layer F.Cu) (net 14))
 (segment (start 110.49 120.65) (end 110.49 131.28) (width 0.25) (layer F.Cu) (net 14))
 (segment (start 142.66 134.24) (end 143.51 134.24) (width 0.25) (layer F.Cu) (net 15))
 (segment (start 139.7 131.28) (end 142.66 134.24) (width 0.25) (layer F.Cu) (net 15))
 (segment (start 139.7 120.65) (end 139.7 131.28) (width 0.25) (layer F.Cu) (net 15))
 (segment (start 174.41 134.24) (end 175.26 134.24) (width 0.25) (layer F.Cu) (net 16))
 (segment (start 171.45 131.28) (end 174.41 134.24) (width 0.25) (layer F.Cu) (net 16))
 (segment (start 171.45 120.65) (end 171.45 131.28) (width 0.25) (layer F.Cu) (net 16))
 (segment (start 85.51 159.64) (end 86.36 159.64) (width 0.25) (layer F.Cu) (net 17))
 (segment (start 82.55 156.68) (end 85.51 159.64) (width 0.25) (layer F.Cu) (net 17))
 (segment (start 82.55 146.05) (end 82.55 156.68) (width 0.25) (layer F.Cu) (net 17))
 (segment (start 175.26 162.94) (end 86.36 162.94) (width 0.25) (layer F.Cu) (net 24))
 (segment (start 204.044999 83.389999) (end 203.195 82.54) (width 0.25) (layer F.Cu) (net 24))
 (segment (start 204.370001 83.715001) (end 204.044999 83.389999) (width 0.25) (layer F.Cu) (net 24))
 (segment (start 204.370001 134.679999) (end 204.370001 83.715001) (width 0.25) (layer F.Cu) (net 24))
 (segment (start 176.11 162.94) (end 204.370001 134.679999) (width 0.25) (layer F.Cu) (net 24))
 (segment (start 175.26 162.94) (end 176.11 162.94) (width 0.25) (layer F.Cu) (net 24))
 (segment (start 110.49 156.68) (end 113.45 159.64) (width 0.25) (layer F.Cu) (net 18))
 (segment (start 113.45 159.64) (end 114.3 159.64) (width 0.25) (layer F.Cu) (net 18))
 (segment (start 110.49 146.05) (end 110.49 156.68) (width 0.25) (layer F.Cu) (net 18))
 (segment (start 141.39 159.64) (end 142.24 159.64) (width 0.25) (layer F.Cu) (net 19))
 (segment (start 138.43 156.68) (end 141.39 159.64) (width 0.25) (layer F.Cu) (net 19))
 (segment (start 138.43 146.05) (end 138.43 156.68) (width 0.25) (layer F.Cu) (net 19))
 (segment (start 174.41 159.64) (end 175.26 159.64) (width 0.25) (layer F.Cu) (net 20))
 (segment (start 171.45 156.68) (end 174.41 159.64) (width 0.25) (layer F.Cu) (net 20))
 (segment (start 171.45 146.05) (end 171.45 156.68) (width 0.25) (layer F.Cu) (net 20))
 (segment (start 88.9 67.31) (end 88.9 63.5) (width 0.25) (layer F.Cu) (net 1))
 (segment (start 88.9 63.5) (end 90.17 62.23) (width 0.25) (layer F.Cu) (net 1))
 (segment (start 182.91 62.23) (end 187.98 67.3) (width 0.25) (layer F.Cu) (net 1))
 (segment (start 90.17 62.23) (end 182.91 62.23) (width 0.25) (layer F.Cu) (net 1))
 (segment (start 88.9 67.31) (end 88.9 143.51) (width 0.25) (layer B.Cu) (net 1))
 (segment (start 185.42 72.36) (end 187.98 74.92) (width 0.25) (layer F.Cu) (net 3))
 (segment (start 185.42 66.04) (end 185.42 72.36) (width 0.25) (layer F.Cu) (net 3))
 (segment (start 116.84 67.31) (end 120.65 63.5) (width 0.25) (layer F.Cu) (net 3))
 (segment (start 182.88 63.5) (end 185.42 66.04) (width 0.25) (layer F.Cu) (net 3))
 (segment (start 120.65 63.5) (end 182.88 63.5) (width 0.25) (layer F.Cu) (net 3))
 (segment (start 116.84 67.31) (end 116.84 143.51) (width 0.25) (layer B.Cu) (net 3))
 (segment (start 184.96999 74.44999) (end 187.98 77.46) (width 0.25) (layer F.Cu) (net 6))
 (segment (start 182.88 64.77) (end 184.96999 66.85999) (width 0.25) (layer F.Cu) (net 6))
 (segment (start 184.96999 66.85999) (end 184.96999 74.44999) (width 0.25) (layer F.Cu) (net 6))
 (segment (start 146.05 67.31) (end 146.05 64.77) (width 0.25) (layer F.Cu) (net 6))
 (segment (start 146.05 64.77) (end 182.88 64.77) (width 0.25) (layer F.Cu) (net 6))
 (segment (start 146.05 142.24) (end 144.78 143.51) (width 0.25) (layer B.Cu) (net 6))
 (segment (start 146.05 67.31) (end 146.05 142.24) (width 0.25) (layer B.Cu) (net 6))
 (segment (start 177.8 143.51) (end 177.8 67.31) (width 0.25) (layer F.Cu) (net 7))
 (segment (start 184.51998 76.53998) (end 187.130001 79.150001) (width 0.25) (layer F.Cu) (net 7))
 (segment (start 187.130001 79.150001) (end 187.98 80) (width 0.25) (layer F.Cu) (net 7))
 (segment (start 184.51998 74.02998) (end 184.51998 76.53998) (width 0.25) (layer F.Cu) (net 7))
 (segment (start 177.8 67.31) (end 184.51998 74.02998) (width 0.25) (layer F.Cu) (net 7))
 (segment (start 187.98 69.84) (end 187.98 72.38) (width 0.25) (layer F.Cu) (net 38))
 (segment (start 201.992919 67.3) (end 203.195 67.3) (width 0.25) (layer F.Cu) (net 38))
 (segment (start 193.860998 67.3) (end 201.992919 67.3) (width 0.25) (layer F.Cu) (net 38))
 (segment (start 191.884999 69.275999) (end 193.860998 67.3) (width 0.25) (layer F.Cu) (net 38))
 (segment (start 191.884999 70.214003) (end 191.884999 69.275999) (width 0.25) (layer F.Cu) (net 38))
 (segment (start 191.084001 71.015001) (end 191.884999 70.214003) (width 0.25) (layer F.Cu) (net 38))
 (segment (start 189.155001 71.015001) (end 191.084001 71.015001) (width 0.25) (layer F.Cu) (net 38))
 (segment (start 187.98 69.84) (end 189.155001 71.015001) (width 0.25) (layer F.Cu) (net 38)))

